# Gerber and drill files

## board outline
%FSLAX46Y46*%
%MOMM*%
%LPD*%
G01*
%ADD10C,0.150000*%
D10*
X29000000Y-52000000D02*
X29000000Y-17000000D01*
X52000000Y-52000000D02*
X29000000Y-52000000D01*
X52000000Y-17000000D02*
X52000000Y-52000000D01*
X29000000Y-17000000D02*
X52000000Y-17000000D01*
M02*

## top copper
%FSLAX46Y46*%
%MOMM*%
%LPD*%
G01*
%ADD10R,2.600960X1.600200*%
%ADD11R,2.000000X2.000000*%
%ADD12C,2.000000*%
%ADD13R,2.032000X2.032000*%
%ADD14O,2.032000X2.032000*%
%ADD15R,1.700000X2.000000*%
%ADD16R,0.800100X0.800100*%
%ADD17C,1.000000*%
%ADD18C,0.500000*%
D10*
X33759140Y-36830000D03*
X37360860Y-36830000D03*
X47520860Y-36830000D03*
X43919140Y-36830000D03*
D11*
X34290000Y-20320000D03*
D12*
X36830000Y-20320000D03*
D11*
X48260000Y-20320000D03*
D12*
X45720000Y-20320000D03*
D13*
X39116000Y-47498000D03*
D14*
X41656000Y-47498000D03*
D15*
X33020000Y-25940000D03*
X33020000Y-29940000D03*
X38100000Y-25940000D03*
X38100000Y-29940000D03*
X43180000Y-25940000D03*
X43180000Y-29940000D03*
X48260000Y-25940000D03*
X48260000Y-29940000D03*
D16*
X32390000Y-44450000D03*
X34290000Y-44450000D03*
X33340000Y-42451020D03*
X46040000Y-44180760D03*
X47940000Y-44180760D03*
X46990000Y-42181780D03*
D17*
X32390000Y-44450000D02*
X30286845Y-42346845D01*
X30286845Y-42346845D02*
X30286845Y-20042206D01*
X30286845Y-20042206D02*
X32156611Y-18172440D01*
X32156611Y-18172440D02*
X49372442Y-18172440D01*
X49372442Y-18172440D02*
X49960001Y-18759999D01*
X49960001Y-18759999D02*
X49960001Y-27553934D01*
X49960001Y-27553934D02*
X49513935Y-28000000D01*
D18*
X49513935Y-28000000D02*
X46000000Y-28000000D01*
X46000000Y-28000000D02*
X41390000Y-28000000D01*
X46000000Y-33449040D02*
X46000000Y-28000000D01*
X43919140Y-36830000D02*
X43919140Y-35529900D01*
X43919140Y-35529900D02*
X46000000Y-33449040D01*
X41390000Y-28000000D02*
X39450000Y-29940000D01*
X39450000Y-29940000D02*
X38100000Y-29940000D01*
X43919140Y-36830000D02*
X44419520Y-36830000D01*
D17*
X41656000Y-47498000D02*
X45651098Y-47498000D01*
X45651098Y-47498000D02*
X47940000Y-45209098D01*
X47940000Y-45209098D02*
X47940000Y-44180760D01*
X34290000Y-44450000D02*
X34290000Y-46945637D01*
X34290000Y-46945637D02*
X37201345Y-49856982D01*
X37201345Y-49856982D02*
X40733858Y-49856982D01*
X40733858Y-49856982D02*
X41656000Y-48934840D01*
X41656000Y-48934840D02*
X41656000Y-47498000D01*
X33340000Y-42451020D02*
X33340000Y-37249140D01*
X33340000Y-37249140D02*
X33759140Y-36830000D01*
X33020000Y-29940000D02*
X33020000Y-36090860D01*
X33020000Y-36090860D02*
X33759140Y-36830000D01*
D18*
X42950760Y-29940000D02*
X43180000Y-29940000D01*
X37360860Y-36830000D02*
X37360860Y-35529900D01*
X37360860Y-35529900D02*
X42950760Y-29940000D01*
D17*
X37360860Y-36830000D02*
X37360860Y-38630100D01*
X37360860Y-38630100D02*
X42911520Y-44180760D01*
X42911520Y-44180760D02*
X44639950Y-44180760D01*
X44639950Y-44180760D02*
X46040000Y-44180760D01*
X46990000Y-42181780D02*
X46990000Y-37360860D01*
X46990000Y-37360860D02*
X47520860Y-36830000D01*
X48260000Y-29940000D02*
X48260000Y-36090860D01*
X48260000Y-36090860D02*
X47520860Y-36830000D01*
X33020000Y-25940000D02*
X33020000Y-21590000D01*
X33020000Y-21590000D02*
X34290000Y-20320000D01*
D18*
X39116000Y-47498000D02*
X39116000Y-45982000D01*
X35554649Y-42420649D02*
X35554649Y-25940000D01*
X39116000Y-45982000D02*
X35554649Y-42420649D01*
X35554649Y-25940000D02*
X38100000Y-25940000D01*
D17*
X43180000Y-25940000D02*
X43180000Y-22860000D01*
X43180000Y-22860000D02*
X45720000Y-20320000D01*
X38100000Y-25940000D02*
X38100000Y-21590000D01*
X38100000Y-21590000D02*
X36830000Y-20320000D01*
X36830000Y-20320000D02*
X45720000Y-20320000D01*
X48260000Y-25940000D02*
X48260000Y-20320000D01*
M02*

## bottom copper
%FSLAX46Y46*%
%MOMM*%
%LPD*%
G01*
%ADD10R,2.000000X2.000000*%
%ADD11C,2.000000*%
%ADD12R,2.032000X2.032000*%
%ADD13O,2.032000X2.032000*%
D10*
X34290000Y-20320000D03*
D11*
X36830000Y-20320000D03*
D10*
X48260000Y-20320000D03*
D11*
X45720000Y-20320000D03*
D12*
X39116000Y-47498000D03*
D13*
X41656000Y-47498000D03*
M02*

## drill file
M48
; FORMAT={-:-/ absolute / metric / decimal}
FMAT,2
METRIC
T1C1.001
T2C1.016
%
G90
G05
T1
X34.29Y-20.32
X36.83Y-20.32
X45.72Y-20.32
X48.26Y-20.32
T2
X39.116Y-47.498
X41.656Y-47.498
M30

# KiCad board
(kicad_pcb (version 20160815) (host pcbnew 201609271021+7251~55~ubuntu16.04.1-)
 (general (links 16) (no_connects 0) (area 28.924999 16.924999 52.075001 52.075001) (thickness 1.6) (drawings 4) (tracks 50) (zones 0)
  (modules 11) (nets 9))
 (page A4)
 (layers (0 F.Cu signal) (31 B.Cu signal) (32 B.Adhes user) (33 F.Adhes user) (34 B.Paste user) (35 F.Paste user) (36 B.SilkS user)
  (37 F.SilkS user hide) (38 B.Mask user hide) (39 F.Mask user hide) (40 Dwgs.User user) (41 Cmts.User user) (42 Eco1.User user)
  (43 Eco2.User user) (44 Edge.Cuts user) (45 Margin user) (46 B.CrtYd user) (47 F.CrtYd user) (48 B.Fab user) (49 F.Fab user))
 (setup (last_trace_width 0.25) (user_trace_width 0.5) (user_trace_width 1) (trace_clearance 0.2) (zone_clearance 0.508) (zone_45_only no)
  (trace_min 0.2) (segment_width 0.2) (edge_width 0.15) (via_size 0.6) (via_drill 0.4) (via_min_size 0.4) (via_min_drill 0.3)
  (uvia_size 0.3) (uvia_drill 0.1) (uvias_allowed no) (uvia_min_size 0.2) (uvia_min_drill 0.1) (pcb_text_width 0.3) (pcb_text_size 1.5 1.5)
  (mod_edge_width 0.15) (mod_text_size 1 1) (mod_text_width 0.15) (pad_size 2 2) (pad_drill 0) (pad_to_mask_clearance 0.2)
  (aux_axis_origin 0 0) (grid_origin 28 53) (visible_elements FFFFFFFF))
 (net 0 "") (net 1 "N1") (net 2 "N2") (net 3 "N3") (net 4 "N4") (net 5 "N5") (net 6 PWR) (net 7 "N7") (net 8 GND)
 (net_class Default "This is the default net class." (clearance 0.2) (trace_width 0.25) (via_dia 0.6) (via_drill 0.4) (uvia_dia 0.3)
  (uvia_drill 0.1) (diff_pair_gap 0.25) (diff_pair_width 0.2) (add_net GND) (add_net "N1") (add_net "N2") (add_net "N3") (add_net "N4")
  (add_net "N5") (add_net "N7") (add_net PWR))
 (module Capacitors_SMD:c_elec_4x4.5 (layer F.Cu) (at 35.56 36.83 180)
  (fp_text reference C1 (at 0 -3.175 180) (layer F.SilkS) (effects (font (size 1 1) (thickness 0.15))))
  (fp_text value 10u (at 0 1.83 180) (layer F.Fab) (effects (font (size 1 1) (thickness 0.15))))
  (pad 1 smd rect (at 1.80086 0 180) (size 2.60096 1.6002) (layers F.Cu F.Paste F.Mask) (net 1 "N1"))
  (pad 2 smd rect (at -1.80086 0 180) (size 2.60096 1.6002) (layers F.Cu F.Paste F.Mask) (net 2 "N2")))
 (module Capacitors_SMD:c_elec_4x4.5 (layer F.Cu) (at 45.72 36.83)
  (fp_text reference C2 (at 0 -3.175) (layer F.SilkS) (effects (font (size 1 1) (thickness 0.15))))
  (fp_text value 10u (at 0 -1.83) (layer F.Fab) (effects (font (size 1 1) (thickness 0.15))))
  (pad 1 smd rect (at 1.80086 0) (size 2.60096 1.6002) (layers F.Cu F.Paste F.Mask) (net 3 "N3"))
  (pad 2 smd rect (at -1.80086 0) (size 2.60096 1.6002) (layers F.Cu F.Paste F.Mask) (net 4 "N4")))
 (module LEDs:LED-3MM (layer F.Cu) (at 34.29 20.32)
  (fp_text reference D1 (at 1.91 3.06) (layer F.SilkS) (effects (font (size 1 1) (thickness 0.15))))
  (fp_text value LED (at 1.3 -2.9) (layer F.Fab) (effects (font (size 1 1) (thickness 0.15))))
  (pad 1 thru_hole rect (at 0 0 90) (size 2 2) (drill 1.00076) (layers *.Cu *.Mask F.SilkS) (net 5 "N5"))
  (pad 2 thru_hole circle (at 2.54 0) (size 2 2) (drill 1.00076) (layers *.Cu *.Mask F.SilkS) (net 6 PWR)))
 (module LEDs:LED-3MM (layer F.Cu) (at 48.26 20.32 180)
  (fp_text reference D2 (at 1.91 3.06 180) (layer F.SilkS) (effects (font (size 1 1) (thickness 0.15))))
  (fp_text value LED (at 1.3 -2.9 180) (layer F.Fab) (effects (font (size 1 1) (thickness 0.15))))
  (pad 1 thru_hole rect (at 0 0 270) (size 2 2) (drill 1.00076) (layers *.Cu *.Mask F.SilkS) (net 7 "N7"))
  (pad 2 thru_hole circle (at 2.54 0 180) (size 2 2) (drill 1.00076) (layers *.Cu *.Mask F.SilkS) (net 6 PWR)))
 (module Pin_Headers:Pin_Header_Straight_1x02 (layer F.Cu) (at 39.116 47.498 90)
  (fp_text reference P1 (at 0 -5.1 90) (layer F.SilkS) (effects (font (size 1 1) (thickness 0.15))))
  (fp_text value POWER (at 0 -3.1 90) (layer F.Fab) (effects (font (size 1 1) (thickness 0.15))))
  (pad 1 thru_hole rect (at 0 0 90) (size 2.032 2.032) (drill 1.016) (layers *.Cu *.Mask F.SilkS) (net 6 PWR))
  (pad 2 thru_hole oval (at 0 2.54 90) (size 2.032 2.032) (drill 1.016) (layers *.Cu *.Mask F.SilkS) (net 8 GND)))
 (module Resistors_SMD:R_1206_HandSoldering (layer F.Cu) (at 33.02 27.94 270)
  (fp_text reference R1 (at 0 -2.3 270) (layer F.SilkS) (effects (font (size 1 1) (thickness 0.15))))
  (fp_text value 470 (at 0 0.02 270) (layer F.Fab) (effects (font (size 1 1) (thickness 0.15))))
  (pad 1 smd rect (at -2 0 270) (size 2 1.7) (layers F.Cu F.Paste F.Mask) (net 5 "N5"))
  (pad 2 smd rect (at 2 0 270) (size 2 1.7) (layers F.Cu F.Paste F.Mask) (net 1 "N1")))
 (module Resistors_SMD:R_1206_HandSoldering (layer F.Cu) (at 38.1 27.94 270)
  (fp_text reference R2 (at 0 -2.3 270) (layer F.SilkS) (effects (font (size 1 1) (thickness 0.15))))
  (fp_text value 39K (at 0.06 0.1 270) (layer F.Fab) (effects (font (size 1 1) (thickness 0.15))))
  (pad 1 smd rect (at -2 0 270) (size 2 1.7) (layers F.Cu F.Paste F.Mask) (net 6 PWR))
  (pad 2 smd rect (at 2 0 270) (size 2 1.7) (layers F.Cu F.Paste F.Mask) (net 4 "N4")))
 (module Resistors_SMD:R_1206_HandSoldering (layer F.Cu) (at 43.18 27.94 270)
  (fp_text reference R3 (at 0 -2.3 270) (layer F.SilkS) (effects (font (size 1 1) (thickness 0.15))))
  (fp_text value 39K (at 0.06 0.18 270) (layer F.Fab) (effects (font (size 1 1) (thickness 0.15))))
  (pad 1 smd rect (at -2 0 270) (size 2 1.7) (layers F.Cu F.Paste F.Mask) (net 6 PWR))
  (pad 2 smd rect (at 2 0 270) (size 2 1.7) (layers F.Cu F.Paste F.Mask) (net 2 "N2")))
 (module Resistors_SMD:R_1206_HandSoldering (layer F.Cu) (at 48.26 27.94 270)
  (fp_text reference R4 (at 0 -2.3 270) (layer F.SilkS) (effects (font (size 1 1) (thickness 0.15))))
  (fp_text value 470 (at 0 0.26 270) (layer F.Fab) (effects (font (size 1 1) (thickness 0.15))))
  (pad 1 smd rect (at -2 0 270) (size 2 1.7) (layers F.Cu F.Paste F.Mask) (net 7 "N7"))
  (pad 2 smd rect (at 2 0 270) (size 2 1.7) (layers F.Cu F.Paste F.Mask) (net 3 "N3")))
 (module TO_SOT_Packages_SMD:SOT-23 (layer F.Cu) (at 33.34 43.44924)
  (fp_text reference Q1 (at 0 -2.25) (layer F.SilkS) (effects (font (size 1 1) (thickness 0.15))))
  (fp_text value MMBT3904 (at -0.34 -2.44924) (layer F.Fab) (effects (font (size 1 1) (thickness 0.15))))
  (pad 1 smd rect (at -0.95 1.00076) (size 0.8001 0.8001) (layers F.Cu F.Paste F.Mask) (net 4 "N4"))
  (pad 2 smd rect (at 0.95 1.00076) (size 0.8001 0.8001) (layers F.Cu F.Paste F.Mask) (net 8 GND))
  (pad 3 smd rect (at 0 -0.99822) (size 0.8001 0.8001) (layers F.Cu F.Paste F.Mask) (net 1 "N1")))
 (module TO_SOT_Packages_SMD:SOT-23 (layer F.Cu) (at 46.99 43.18)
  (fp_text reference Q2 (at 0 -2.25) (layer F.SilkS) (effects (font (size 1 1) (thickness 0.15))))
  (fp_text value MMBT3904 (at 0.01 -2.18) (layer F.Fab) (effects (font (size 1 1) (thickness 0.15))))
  (pad 1 smd rect (at -0.95 1.00076) (size 0.8001 0.8001) (layers F.Cu F.Paste F.Mask) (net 2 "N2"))
  (pad 2 smd rect (at 0.95 1.00076) (size 0.8001 0.8001) (layers F.Cu F.Paste F.Mask) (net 8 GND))
  (pad 3 smd rect (at 0 -0.99822) (size 0.8001 0.8001) (layers F.Cu F.Paste F.Mask) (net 3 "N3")))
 (gr_line (start 29 52) (end 29 17) (layer Edge.Cuts) (width 0.15))
 (gr_line (start 52 52) (end 29 52) (layer Edge.Cuts) (width 0.15))
 (gr_line (start 52 17) (end 52 52) (layer Edge.Cuts) (width 0.15))
 (gr_line (start 29 17) (end 52 17) (layer Edge.Cuts) (width 0.15))
 (segment (start 32.39 44.45) (end 30.286845 42.346845) (width 1) (layer F.Cu) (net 4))
 (segment (start 30.286845 42.346845) (end 30.286845 20.042206) (width 1) (layer F.Cu) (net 4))
 (segment (start 30.286845 20.042206) (end 32.156611 18.17244) (width 1) (layer F.Cu) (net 4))
 (segment (start 32.156611 18.17244) (end 49.372442 18.17244) (width 1) (layer F.Cu) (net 4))
 (segment (start 49.372442 18.17244) (end 49.960001 18.759999) (width 1) (layer F.Cu) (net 4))
 (segment (start 49.960001 18.759999) (end 49.960001 27.553934) (width 1) (layer F.Cu) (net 4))
 (segment (start 49.960001 27.553934) (end 49.513935 28) (width 1) (layer F.Cu) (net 4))
 (segment (start 49.513935 28) (end 46 28) (width 0.5) (layer F.Cu) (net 4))
 (segment (start 46 28) (end 41.39 28) (width 0.5) (layer F.Cu) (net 4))
 (segment (start 46 33.44904) (end 46 28) (width 0.5) (layer F.Cu) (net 4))
 (segment (start 43.91914 36.83) (end 43.91914 35.5299) (width 0.5) (layer F.Cu) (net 4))
 (segment (start 43.91914 35.5299) (end 46 33.44904) (width 0.5) (layer F.Cu) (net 4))
 (segment (start 41.39 28) (end 39.45 29.94) (width 0.5) (layer F.Cu) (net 4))
 (segment (start 39.45 29.94) (end 38.1 29.94) (width 0.5) (layer F.Cu) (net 4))
 (segment (start 43.91914 36.83) (end 44.41952 36.83) (width 0.5) (layer F.Cu) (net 4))
 (segment (start 41.656 47.498) (end 45.651098 47.498) (width 1) (layer F.Cu) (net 8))
 (segment (start 45.651098 47.498) (end 47.94 45.209098) (width 1) (layer F.Cu) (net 8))
 (segment (start 47.94 45.209098) (end 47.94 44.18076) (width 1) (layer F.Cu) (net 8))
 (segment (start 34.29 44.45) (end 34.29 46.945637) (width 1) (layer F.Cu) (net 8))
 (segment (start 34.29 46.945637) (end 37.201345 49.856982) (width 1) (layer F.Cu) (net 8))
 (segment (start 37.201345 49.856982) (end 40.733858 49.856982) (width 1) (layer F.Cu) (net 8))
 (segment (start 40.733858 49.856982) (end 41.656 48.93484) (width 1) (layer F.Cu) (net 8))
 (segment (start 41.656 48.93484) (end 41.656 47.498) (width 1) (layer F.Cu) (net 8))
 (segment (start 33.34 42.45102) (end 33.34 37.24914) (width 1) (layer F.Cu) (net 1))
 (segment (start 33.34 37.24914) (end 33.75914 36.83) (width 1) (layer F.Cu) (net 1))
 (segment (start 33.02 29.94) (end 33.02 36.09086) (width 1) (layer F.Cu) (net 1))
 (segment (start 33.02 36.09086) (end 33.75914 36.83) (width 1) (layer F.Cu) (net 1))
 (segment (start 42.95076 29.94) (end 43.18 29.94) (width 0.5) (layer F.Cu) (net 2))
 (segment (start 37.36086 36.83) (end 37.36086 35.5299) (width 0.5) (layer F.Cu) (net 2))
 (segment (start 37.36086 35.5299) (end 42.95076 29.94) (width 0.5) (layer F.Cu) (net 2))
 (segment (start 37.36086 36.83) (end 37.36086 38.6301) (width 1) (layer F.Cu) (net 2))
 (segment (start 37.36086 38.6301) (end 42.91152 44.18076) (width 1) (layer F.Cu) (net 2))
 (segment (start 42.91152 44.18076) (end 44.63995 44.18076) (width 1) (layer F.Cu) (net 2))
 (segment (start 44.63995 44.18076) (end 46.04 44.18076) (width 1) (layer F.Cu) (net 2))
 (segment (start 46.99 42.18178) (end 46.99 37.36086) (width 1) (layer F.Cu) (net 3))
 (segment (start 46.99 37.36086) (end 47.52086 36.83) (width 1) (layer F.Cu) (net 3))
 (segment (start 48.26 29.94) (end 48.26 36.09086) (width 1) (layer F.Cu) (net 3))
 (segment (start 48.26 36.09086) (end 47.52086 36.83) (width 1) (layer F.Cu) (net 3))
 (segment (start 33.02 25.94) (end 33.02 21.59) (width 1) (layer F.Cu) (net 5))
 (segment (start 33.02 21.59) (end 34.29 20.32) (width 1) (layer F.Cu) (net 5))
 (segment (start 39.116 47.498) (end 39.116 45.982) (width 0.5) (layer F.Cu) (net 6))
 (segment (start 35.554649 42.420649) (end 35.554649 25.94) (width 0.5) (layer F.Cu) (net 6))
 (segment (start 39.116 45.982) (end 35.554649 42.420649) (width 0.5) (layer F.Cu) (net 6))
 (segment (start 35.554649 25.94) (end 38.1 25.94) (width 0.5) (layer F.Cu) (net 6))
 (segment (start 43.18 25.94) (end 43.18 22.86) (width 1) (layer F.Cu) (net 6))
 (segment (start 43.18 22.86) (end 45.72 20.32) (width 1) (layer F.Cu) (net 6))
 (segment (start 38.1 25.94) (end 38.1 21.59) (width 1) (layer F.Cu) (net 6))
 (segment (start 38.1 21.59) (end 36.83 20.32) (width 1) (layer F.Cu) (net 6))
 (segment (start 36.83 20.32) (end 45.72 20.32) (width 1) (layer F.Cu) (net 6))
 (segment (start 48.26 25.94) (end 48.26 20.32) (width 1) (layer F.Cu) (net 7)))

